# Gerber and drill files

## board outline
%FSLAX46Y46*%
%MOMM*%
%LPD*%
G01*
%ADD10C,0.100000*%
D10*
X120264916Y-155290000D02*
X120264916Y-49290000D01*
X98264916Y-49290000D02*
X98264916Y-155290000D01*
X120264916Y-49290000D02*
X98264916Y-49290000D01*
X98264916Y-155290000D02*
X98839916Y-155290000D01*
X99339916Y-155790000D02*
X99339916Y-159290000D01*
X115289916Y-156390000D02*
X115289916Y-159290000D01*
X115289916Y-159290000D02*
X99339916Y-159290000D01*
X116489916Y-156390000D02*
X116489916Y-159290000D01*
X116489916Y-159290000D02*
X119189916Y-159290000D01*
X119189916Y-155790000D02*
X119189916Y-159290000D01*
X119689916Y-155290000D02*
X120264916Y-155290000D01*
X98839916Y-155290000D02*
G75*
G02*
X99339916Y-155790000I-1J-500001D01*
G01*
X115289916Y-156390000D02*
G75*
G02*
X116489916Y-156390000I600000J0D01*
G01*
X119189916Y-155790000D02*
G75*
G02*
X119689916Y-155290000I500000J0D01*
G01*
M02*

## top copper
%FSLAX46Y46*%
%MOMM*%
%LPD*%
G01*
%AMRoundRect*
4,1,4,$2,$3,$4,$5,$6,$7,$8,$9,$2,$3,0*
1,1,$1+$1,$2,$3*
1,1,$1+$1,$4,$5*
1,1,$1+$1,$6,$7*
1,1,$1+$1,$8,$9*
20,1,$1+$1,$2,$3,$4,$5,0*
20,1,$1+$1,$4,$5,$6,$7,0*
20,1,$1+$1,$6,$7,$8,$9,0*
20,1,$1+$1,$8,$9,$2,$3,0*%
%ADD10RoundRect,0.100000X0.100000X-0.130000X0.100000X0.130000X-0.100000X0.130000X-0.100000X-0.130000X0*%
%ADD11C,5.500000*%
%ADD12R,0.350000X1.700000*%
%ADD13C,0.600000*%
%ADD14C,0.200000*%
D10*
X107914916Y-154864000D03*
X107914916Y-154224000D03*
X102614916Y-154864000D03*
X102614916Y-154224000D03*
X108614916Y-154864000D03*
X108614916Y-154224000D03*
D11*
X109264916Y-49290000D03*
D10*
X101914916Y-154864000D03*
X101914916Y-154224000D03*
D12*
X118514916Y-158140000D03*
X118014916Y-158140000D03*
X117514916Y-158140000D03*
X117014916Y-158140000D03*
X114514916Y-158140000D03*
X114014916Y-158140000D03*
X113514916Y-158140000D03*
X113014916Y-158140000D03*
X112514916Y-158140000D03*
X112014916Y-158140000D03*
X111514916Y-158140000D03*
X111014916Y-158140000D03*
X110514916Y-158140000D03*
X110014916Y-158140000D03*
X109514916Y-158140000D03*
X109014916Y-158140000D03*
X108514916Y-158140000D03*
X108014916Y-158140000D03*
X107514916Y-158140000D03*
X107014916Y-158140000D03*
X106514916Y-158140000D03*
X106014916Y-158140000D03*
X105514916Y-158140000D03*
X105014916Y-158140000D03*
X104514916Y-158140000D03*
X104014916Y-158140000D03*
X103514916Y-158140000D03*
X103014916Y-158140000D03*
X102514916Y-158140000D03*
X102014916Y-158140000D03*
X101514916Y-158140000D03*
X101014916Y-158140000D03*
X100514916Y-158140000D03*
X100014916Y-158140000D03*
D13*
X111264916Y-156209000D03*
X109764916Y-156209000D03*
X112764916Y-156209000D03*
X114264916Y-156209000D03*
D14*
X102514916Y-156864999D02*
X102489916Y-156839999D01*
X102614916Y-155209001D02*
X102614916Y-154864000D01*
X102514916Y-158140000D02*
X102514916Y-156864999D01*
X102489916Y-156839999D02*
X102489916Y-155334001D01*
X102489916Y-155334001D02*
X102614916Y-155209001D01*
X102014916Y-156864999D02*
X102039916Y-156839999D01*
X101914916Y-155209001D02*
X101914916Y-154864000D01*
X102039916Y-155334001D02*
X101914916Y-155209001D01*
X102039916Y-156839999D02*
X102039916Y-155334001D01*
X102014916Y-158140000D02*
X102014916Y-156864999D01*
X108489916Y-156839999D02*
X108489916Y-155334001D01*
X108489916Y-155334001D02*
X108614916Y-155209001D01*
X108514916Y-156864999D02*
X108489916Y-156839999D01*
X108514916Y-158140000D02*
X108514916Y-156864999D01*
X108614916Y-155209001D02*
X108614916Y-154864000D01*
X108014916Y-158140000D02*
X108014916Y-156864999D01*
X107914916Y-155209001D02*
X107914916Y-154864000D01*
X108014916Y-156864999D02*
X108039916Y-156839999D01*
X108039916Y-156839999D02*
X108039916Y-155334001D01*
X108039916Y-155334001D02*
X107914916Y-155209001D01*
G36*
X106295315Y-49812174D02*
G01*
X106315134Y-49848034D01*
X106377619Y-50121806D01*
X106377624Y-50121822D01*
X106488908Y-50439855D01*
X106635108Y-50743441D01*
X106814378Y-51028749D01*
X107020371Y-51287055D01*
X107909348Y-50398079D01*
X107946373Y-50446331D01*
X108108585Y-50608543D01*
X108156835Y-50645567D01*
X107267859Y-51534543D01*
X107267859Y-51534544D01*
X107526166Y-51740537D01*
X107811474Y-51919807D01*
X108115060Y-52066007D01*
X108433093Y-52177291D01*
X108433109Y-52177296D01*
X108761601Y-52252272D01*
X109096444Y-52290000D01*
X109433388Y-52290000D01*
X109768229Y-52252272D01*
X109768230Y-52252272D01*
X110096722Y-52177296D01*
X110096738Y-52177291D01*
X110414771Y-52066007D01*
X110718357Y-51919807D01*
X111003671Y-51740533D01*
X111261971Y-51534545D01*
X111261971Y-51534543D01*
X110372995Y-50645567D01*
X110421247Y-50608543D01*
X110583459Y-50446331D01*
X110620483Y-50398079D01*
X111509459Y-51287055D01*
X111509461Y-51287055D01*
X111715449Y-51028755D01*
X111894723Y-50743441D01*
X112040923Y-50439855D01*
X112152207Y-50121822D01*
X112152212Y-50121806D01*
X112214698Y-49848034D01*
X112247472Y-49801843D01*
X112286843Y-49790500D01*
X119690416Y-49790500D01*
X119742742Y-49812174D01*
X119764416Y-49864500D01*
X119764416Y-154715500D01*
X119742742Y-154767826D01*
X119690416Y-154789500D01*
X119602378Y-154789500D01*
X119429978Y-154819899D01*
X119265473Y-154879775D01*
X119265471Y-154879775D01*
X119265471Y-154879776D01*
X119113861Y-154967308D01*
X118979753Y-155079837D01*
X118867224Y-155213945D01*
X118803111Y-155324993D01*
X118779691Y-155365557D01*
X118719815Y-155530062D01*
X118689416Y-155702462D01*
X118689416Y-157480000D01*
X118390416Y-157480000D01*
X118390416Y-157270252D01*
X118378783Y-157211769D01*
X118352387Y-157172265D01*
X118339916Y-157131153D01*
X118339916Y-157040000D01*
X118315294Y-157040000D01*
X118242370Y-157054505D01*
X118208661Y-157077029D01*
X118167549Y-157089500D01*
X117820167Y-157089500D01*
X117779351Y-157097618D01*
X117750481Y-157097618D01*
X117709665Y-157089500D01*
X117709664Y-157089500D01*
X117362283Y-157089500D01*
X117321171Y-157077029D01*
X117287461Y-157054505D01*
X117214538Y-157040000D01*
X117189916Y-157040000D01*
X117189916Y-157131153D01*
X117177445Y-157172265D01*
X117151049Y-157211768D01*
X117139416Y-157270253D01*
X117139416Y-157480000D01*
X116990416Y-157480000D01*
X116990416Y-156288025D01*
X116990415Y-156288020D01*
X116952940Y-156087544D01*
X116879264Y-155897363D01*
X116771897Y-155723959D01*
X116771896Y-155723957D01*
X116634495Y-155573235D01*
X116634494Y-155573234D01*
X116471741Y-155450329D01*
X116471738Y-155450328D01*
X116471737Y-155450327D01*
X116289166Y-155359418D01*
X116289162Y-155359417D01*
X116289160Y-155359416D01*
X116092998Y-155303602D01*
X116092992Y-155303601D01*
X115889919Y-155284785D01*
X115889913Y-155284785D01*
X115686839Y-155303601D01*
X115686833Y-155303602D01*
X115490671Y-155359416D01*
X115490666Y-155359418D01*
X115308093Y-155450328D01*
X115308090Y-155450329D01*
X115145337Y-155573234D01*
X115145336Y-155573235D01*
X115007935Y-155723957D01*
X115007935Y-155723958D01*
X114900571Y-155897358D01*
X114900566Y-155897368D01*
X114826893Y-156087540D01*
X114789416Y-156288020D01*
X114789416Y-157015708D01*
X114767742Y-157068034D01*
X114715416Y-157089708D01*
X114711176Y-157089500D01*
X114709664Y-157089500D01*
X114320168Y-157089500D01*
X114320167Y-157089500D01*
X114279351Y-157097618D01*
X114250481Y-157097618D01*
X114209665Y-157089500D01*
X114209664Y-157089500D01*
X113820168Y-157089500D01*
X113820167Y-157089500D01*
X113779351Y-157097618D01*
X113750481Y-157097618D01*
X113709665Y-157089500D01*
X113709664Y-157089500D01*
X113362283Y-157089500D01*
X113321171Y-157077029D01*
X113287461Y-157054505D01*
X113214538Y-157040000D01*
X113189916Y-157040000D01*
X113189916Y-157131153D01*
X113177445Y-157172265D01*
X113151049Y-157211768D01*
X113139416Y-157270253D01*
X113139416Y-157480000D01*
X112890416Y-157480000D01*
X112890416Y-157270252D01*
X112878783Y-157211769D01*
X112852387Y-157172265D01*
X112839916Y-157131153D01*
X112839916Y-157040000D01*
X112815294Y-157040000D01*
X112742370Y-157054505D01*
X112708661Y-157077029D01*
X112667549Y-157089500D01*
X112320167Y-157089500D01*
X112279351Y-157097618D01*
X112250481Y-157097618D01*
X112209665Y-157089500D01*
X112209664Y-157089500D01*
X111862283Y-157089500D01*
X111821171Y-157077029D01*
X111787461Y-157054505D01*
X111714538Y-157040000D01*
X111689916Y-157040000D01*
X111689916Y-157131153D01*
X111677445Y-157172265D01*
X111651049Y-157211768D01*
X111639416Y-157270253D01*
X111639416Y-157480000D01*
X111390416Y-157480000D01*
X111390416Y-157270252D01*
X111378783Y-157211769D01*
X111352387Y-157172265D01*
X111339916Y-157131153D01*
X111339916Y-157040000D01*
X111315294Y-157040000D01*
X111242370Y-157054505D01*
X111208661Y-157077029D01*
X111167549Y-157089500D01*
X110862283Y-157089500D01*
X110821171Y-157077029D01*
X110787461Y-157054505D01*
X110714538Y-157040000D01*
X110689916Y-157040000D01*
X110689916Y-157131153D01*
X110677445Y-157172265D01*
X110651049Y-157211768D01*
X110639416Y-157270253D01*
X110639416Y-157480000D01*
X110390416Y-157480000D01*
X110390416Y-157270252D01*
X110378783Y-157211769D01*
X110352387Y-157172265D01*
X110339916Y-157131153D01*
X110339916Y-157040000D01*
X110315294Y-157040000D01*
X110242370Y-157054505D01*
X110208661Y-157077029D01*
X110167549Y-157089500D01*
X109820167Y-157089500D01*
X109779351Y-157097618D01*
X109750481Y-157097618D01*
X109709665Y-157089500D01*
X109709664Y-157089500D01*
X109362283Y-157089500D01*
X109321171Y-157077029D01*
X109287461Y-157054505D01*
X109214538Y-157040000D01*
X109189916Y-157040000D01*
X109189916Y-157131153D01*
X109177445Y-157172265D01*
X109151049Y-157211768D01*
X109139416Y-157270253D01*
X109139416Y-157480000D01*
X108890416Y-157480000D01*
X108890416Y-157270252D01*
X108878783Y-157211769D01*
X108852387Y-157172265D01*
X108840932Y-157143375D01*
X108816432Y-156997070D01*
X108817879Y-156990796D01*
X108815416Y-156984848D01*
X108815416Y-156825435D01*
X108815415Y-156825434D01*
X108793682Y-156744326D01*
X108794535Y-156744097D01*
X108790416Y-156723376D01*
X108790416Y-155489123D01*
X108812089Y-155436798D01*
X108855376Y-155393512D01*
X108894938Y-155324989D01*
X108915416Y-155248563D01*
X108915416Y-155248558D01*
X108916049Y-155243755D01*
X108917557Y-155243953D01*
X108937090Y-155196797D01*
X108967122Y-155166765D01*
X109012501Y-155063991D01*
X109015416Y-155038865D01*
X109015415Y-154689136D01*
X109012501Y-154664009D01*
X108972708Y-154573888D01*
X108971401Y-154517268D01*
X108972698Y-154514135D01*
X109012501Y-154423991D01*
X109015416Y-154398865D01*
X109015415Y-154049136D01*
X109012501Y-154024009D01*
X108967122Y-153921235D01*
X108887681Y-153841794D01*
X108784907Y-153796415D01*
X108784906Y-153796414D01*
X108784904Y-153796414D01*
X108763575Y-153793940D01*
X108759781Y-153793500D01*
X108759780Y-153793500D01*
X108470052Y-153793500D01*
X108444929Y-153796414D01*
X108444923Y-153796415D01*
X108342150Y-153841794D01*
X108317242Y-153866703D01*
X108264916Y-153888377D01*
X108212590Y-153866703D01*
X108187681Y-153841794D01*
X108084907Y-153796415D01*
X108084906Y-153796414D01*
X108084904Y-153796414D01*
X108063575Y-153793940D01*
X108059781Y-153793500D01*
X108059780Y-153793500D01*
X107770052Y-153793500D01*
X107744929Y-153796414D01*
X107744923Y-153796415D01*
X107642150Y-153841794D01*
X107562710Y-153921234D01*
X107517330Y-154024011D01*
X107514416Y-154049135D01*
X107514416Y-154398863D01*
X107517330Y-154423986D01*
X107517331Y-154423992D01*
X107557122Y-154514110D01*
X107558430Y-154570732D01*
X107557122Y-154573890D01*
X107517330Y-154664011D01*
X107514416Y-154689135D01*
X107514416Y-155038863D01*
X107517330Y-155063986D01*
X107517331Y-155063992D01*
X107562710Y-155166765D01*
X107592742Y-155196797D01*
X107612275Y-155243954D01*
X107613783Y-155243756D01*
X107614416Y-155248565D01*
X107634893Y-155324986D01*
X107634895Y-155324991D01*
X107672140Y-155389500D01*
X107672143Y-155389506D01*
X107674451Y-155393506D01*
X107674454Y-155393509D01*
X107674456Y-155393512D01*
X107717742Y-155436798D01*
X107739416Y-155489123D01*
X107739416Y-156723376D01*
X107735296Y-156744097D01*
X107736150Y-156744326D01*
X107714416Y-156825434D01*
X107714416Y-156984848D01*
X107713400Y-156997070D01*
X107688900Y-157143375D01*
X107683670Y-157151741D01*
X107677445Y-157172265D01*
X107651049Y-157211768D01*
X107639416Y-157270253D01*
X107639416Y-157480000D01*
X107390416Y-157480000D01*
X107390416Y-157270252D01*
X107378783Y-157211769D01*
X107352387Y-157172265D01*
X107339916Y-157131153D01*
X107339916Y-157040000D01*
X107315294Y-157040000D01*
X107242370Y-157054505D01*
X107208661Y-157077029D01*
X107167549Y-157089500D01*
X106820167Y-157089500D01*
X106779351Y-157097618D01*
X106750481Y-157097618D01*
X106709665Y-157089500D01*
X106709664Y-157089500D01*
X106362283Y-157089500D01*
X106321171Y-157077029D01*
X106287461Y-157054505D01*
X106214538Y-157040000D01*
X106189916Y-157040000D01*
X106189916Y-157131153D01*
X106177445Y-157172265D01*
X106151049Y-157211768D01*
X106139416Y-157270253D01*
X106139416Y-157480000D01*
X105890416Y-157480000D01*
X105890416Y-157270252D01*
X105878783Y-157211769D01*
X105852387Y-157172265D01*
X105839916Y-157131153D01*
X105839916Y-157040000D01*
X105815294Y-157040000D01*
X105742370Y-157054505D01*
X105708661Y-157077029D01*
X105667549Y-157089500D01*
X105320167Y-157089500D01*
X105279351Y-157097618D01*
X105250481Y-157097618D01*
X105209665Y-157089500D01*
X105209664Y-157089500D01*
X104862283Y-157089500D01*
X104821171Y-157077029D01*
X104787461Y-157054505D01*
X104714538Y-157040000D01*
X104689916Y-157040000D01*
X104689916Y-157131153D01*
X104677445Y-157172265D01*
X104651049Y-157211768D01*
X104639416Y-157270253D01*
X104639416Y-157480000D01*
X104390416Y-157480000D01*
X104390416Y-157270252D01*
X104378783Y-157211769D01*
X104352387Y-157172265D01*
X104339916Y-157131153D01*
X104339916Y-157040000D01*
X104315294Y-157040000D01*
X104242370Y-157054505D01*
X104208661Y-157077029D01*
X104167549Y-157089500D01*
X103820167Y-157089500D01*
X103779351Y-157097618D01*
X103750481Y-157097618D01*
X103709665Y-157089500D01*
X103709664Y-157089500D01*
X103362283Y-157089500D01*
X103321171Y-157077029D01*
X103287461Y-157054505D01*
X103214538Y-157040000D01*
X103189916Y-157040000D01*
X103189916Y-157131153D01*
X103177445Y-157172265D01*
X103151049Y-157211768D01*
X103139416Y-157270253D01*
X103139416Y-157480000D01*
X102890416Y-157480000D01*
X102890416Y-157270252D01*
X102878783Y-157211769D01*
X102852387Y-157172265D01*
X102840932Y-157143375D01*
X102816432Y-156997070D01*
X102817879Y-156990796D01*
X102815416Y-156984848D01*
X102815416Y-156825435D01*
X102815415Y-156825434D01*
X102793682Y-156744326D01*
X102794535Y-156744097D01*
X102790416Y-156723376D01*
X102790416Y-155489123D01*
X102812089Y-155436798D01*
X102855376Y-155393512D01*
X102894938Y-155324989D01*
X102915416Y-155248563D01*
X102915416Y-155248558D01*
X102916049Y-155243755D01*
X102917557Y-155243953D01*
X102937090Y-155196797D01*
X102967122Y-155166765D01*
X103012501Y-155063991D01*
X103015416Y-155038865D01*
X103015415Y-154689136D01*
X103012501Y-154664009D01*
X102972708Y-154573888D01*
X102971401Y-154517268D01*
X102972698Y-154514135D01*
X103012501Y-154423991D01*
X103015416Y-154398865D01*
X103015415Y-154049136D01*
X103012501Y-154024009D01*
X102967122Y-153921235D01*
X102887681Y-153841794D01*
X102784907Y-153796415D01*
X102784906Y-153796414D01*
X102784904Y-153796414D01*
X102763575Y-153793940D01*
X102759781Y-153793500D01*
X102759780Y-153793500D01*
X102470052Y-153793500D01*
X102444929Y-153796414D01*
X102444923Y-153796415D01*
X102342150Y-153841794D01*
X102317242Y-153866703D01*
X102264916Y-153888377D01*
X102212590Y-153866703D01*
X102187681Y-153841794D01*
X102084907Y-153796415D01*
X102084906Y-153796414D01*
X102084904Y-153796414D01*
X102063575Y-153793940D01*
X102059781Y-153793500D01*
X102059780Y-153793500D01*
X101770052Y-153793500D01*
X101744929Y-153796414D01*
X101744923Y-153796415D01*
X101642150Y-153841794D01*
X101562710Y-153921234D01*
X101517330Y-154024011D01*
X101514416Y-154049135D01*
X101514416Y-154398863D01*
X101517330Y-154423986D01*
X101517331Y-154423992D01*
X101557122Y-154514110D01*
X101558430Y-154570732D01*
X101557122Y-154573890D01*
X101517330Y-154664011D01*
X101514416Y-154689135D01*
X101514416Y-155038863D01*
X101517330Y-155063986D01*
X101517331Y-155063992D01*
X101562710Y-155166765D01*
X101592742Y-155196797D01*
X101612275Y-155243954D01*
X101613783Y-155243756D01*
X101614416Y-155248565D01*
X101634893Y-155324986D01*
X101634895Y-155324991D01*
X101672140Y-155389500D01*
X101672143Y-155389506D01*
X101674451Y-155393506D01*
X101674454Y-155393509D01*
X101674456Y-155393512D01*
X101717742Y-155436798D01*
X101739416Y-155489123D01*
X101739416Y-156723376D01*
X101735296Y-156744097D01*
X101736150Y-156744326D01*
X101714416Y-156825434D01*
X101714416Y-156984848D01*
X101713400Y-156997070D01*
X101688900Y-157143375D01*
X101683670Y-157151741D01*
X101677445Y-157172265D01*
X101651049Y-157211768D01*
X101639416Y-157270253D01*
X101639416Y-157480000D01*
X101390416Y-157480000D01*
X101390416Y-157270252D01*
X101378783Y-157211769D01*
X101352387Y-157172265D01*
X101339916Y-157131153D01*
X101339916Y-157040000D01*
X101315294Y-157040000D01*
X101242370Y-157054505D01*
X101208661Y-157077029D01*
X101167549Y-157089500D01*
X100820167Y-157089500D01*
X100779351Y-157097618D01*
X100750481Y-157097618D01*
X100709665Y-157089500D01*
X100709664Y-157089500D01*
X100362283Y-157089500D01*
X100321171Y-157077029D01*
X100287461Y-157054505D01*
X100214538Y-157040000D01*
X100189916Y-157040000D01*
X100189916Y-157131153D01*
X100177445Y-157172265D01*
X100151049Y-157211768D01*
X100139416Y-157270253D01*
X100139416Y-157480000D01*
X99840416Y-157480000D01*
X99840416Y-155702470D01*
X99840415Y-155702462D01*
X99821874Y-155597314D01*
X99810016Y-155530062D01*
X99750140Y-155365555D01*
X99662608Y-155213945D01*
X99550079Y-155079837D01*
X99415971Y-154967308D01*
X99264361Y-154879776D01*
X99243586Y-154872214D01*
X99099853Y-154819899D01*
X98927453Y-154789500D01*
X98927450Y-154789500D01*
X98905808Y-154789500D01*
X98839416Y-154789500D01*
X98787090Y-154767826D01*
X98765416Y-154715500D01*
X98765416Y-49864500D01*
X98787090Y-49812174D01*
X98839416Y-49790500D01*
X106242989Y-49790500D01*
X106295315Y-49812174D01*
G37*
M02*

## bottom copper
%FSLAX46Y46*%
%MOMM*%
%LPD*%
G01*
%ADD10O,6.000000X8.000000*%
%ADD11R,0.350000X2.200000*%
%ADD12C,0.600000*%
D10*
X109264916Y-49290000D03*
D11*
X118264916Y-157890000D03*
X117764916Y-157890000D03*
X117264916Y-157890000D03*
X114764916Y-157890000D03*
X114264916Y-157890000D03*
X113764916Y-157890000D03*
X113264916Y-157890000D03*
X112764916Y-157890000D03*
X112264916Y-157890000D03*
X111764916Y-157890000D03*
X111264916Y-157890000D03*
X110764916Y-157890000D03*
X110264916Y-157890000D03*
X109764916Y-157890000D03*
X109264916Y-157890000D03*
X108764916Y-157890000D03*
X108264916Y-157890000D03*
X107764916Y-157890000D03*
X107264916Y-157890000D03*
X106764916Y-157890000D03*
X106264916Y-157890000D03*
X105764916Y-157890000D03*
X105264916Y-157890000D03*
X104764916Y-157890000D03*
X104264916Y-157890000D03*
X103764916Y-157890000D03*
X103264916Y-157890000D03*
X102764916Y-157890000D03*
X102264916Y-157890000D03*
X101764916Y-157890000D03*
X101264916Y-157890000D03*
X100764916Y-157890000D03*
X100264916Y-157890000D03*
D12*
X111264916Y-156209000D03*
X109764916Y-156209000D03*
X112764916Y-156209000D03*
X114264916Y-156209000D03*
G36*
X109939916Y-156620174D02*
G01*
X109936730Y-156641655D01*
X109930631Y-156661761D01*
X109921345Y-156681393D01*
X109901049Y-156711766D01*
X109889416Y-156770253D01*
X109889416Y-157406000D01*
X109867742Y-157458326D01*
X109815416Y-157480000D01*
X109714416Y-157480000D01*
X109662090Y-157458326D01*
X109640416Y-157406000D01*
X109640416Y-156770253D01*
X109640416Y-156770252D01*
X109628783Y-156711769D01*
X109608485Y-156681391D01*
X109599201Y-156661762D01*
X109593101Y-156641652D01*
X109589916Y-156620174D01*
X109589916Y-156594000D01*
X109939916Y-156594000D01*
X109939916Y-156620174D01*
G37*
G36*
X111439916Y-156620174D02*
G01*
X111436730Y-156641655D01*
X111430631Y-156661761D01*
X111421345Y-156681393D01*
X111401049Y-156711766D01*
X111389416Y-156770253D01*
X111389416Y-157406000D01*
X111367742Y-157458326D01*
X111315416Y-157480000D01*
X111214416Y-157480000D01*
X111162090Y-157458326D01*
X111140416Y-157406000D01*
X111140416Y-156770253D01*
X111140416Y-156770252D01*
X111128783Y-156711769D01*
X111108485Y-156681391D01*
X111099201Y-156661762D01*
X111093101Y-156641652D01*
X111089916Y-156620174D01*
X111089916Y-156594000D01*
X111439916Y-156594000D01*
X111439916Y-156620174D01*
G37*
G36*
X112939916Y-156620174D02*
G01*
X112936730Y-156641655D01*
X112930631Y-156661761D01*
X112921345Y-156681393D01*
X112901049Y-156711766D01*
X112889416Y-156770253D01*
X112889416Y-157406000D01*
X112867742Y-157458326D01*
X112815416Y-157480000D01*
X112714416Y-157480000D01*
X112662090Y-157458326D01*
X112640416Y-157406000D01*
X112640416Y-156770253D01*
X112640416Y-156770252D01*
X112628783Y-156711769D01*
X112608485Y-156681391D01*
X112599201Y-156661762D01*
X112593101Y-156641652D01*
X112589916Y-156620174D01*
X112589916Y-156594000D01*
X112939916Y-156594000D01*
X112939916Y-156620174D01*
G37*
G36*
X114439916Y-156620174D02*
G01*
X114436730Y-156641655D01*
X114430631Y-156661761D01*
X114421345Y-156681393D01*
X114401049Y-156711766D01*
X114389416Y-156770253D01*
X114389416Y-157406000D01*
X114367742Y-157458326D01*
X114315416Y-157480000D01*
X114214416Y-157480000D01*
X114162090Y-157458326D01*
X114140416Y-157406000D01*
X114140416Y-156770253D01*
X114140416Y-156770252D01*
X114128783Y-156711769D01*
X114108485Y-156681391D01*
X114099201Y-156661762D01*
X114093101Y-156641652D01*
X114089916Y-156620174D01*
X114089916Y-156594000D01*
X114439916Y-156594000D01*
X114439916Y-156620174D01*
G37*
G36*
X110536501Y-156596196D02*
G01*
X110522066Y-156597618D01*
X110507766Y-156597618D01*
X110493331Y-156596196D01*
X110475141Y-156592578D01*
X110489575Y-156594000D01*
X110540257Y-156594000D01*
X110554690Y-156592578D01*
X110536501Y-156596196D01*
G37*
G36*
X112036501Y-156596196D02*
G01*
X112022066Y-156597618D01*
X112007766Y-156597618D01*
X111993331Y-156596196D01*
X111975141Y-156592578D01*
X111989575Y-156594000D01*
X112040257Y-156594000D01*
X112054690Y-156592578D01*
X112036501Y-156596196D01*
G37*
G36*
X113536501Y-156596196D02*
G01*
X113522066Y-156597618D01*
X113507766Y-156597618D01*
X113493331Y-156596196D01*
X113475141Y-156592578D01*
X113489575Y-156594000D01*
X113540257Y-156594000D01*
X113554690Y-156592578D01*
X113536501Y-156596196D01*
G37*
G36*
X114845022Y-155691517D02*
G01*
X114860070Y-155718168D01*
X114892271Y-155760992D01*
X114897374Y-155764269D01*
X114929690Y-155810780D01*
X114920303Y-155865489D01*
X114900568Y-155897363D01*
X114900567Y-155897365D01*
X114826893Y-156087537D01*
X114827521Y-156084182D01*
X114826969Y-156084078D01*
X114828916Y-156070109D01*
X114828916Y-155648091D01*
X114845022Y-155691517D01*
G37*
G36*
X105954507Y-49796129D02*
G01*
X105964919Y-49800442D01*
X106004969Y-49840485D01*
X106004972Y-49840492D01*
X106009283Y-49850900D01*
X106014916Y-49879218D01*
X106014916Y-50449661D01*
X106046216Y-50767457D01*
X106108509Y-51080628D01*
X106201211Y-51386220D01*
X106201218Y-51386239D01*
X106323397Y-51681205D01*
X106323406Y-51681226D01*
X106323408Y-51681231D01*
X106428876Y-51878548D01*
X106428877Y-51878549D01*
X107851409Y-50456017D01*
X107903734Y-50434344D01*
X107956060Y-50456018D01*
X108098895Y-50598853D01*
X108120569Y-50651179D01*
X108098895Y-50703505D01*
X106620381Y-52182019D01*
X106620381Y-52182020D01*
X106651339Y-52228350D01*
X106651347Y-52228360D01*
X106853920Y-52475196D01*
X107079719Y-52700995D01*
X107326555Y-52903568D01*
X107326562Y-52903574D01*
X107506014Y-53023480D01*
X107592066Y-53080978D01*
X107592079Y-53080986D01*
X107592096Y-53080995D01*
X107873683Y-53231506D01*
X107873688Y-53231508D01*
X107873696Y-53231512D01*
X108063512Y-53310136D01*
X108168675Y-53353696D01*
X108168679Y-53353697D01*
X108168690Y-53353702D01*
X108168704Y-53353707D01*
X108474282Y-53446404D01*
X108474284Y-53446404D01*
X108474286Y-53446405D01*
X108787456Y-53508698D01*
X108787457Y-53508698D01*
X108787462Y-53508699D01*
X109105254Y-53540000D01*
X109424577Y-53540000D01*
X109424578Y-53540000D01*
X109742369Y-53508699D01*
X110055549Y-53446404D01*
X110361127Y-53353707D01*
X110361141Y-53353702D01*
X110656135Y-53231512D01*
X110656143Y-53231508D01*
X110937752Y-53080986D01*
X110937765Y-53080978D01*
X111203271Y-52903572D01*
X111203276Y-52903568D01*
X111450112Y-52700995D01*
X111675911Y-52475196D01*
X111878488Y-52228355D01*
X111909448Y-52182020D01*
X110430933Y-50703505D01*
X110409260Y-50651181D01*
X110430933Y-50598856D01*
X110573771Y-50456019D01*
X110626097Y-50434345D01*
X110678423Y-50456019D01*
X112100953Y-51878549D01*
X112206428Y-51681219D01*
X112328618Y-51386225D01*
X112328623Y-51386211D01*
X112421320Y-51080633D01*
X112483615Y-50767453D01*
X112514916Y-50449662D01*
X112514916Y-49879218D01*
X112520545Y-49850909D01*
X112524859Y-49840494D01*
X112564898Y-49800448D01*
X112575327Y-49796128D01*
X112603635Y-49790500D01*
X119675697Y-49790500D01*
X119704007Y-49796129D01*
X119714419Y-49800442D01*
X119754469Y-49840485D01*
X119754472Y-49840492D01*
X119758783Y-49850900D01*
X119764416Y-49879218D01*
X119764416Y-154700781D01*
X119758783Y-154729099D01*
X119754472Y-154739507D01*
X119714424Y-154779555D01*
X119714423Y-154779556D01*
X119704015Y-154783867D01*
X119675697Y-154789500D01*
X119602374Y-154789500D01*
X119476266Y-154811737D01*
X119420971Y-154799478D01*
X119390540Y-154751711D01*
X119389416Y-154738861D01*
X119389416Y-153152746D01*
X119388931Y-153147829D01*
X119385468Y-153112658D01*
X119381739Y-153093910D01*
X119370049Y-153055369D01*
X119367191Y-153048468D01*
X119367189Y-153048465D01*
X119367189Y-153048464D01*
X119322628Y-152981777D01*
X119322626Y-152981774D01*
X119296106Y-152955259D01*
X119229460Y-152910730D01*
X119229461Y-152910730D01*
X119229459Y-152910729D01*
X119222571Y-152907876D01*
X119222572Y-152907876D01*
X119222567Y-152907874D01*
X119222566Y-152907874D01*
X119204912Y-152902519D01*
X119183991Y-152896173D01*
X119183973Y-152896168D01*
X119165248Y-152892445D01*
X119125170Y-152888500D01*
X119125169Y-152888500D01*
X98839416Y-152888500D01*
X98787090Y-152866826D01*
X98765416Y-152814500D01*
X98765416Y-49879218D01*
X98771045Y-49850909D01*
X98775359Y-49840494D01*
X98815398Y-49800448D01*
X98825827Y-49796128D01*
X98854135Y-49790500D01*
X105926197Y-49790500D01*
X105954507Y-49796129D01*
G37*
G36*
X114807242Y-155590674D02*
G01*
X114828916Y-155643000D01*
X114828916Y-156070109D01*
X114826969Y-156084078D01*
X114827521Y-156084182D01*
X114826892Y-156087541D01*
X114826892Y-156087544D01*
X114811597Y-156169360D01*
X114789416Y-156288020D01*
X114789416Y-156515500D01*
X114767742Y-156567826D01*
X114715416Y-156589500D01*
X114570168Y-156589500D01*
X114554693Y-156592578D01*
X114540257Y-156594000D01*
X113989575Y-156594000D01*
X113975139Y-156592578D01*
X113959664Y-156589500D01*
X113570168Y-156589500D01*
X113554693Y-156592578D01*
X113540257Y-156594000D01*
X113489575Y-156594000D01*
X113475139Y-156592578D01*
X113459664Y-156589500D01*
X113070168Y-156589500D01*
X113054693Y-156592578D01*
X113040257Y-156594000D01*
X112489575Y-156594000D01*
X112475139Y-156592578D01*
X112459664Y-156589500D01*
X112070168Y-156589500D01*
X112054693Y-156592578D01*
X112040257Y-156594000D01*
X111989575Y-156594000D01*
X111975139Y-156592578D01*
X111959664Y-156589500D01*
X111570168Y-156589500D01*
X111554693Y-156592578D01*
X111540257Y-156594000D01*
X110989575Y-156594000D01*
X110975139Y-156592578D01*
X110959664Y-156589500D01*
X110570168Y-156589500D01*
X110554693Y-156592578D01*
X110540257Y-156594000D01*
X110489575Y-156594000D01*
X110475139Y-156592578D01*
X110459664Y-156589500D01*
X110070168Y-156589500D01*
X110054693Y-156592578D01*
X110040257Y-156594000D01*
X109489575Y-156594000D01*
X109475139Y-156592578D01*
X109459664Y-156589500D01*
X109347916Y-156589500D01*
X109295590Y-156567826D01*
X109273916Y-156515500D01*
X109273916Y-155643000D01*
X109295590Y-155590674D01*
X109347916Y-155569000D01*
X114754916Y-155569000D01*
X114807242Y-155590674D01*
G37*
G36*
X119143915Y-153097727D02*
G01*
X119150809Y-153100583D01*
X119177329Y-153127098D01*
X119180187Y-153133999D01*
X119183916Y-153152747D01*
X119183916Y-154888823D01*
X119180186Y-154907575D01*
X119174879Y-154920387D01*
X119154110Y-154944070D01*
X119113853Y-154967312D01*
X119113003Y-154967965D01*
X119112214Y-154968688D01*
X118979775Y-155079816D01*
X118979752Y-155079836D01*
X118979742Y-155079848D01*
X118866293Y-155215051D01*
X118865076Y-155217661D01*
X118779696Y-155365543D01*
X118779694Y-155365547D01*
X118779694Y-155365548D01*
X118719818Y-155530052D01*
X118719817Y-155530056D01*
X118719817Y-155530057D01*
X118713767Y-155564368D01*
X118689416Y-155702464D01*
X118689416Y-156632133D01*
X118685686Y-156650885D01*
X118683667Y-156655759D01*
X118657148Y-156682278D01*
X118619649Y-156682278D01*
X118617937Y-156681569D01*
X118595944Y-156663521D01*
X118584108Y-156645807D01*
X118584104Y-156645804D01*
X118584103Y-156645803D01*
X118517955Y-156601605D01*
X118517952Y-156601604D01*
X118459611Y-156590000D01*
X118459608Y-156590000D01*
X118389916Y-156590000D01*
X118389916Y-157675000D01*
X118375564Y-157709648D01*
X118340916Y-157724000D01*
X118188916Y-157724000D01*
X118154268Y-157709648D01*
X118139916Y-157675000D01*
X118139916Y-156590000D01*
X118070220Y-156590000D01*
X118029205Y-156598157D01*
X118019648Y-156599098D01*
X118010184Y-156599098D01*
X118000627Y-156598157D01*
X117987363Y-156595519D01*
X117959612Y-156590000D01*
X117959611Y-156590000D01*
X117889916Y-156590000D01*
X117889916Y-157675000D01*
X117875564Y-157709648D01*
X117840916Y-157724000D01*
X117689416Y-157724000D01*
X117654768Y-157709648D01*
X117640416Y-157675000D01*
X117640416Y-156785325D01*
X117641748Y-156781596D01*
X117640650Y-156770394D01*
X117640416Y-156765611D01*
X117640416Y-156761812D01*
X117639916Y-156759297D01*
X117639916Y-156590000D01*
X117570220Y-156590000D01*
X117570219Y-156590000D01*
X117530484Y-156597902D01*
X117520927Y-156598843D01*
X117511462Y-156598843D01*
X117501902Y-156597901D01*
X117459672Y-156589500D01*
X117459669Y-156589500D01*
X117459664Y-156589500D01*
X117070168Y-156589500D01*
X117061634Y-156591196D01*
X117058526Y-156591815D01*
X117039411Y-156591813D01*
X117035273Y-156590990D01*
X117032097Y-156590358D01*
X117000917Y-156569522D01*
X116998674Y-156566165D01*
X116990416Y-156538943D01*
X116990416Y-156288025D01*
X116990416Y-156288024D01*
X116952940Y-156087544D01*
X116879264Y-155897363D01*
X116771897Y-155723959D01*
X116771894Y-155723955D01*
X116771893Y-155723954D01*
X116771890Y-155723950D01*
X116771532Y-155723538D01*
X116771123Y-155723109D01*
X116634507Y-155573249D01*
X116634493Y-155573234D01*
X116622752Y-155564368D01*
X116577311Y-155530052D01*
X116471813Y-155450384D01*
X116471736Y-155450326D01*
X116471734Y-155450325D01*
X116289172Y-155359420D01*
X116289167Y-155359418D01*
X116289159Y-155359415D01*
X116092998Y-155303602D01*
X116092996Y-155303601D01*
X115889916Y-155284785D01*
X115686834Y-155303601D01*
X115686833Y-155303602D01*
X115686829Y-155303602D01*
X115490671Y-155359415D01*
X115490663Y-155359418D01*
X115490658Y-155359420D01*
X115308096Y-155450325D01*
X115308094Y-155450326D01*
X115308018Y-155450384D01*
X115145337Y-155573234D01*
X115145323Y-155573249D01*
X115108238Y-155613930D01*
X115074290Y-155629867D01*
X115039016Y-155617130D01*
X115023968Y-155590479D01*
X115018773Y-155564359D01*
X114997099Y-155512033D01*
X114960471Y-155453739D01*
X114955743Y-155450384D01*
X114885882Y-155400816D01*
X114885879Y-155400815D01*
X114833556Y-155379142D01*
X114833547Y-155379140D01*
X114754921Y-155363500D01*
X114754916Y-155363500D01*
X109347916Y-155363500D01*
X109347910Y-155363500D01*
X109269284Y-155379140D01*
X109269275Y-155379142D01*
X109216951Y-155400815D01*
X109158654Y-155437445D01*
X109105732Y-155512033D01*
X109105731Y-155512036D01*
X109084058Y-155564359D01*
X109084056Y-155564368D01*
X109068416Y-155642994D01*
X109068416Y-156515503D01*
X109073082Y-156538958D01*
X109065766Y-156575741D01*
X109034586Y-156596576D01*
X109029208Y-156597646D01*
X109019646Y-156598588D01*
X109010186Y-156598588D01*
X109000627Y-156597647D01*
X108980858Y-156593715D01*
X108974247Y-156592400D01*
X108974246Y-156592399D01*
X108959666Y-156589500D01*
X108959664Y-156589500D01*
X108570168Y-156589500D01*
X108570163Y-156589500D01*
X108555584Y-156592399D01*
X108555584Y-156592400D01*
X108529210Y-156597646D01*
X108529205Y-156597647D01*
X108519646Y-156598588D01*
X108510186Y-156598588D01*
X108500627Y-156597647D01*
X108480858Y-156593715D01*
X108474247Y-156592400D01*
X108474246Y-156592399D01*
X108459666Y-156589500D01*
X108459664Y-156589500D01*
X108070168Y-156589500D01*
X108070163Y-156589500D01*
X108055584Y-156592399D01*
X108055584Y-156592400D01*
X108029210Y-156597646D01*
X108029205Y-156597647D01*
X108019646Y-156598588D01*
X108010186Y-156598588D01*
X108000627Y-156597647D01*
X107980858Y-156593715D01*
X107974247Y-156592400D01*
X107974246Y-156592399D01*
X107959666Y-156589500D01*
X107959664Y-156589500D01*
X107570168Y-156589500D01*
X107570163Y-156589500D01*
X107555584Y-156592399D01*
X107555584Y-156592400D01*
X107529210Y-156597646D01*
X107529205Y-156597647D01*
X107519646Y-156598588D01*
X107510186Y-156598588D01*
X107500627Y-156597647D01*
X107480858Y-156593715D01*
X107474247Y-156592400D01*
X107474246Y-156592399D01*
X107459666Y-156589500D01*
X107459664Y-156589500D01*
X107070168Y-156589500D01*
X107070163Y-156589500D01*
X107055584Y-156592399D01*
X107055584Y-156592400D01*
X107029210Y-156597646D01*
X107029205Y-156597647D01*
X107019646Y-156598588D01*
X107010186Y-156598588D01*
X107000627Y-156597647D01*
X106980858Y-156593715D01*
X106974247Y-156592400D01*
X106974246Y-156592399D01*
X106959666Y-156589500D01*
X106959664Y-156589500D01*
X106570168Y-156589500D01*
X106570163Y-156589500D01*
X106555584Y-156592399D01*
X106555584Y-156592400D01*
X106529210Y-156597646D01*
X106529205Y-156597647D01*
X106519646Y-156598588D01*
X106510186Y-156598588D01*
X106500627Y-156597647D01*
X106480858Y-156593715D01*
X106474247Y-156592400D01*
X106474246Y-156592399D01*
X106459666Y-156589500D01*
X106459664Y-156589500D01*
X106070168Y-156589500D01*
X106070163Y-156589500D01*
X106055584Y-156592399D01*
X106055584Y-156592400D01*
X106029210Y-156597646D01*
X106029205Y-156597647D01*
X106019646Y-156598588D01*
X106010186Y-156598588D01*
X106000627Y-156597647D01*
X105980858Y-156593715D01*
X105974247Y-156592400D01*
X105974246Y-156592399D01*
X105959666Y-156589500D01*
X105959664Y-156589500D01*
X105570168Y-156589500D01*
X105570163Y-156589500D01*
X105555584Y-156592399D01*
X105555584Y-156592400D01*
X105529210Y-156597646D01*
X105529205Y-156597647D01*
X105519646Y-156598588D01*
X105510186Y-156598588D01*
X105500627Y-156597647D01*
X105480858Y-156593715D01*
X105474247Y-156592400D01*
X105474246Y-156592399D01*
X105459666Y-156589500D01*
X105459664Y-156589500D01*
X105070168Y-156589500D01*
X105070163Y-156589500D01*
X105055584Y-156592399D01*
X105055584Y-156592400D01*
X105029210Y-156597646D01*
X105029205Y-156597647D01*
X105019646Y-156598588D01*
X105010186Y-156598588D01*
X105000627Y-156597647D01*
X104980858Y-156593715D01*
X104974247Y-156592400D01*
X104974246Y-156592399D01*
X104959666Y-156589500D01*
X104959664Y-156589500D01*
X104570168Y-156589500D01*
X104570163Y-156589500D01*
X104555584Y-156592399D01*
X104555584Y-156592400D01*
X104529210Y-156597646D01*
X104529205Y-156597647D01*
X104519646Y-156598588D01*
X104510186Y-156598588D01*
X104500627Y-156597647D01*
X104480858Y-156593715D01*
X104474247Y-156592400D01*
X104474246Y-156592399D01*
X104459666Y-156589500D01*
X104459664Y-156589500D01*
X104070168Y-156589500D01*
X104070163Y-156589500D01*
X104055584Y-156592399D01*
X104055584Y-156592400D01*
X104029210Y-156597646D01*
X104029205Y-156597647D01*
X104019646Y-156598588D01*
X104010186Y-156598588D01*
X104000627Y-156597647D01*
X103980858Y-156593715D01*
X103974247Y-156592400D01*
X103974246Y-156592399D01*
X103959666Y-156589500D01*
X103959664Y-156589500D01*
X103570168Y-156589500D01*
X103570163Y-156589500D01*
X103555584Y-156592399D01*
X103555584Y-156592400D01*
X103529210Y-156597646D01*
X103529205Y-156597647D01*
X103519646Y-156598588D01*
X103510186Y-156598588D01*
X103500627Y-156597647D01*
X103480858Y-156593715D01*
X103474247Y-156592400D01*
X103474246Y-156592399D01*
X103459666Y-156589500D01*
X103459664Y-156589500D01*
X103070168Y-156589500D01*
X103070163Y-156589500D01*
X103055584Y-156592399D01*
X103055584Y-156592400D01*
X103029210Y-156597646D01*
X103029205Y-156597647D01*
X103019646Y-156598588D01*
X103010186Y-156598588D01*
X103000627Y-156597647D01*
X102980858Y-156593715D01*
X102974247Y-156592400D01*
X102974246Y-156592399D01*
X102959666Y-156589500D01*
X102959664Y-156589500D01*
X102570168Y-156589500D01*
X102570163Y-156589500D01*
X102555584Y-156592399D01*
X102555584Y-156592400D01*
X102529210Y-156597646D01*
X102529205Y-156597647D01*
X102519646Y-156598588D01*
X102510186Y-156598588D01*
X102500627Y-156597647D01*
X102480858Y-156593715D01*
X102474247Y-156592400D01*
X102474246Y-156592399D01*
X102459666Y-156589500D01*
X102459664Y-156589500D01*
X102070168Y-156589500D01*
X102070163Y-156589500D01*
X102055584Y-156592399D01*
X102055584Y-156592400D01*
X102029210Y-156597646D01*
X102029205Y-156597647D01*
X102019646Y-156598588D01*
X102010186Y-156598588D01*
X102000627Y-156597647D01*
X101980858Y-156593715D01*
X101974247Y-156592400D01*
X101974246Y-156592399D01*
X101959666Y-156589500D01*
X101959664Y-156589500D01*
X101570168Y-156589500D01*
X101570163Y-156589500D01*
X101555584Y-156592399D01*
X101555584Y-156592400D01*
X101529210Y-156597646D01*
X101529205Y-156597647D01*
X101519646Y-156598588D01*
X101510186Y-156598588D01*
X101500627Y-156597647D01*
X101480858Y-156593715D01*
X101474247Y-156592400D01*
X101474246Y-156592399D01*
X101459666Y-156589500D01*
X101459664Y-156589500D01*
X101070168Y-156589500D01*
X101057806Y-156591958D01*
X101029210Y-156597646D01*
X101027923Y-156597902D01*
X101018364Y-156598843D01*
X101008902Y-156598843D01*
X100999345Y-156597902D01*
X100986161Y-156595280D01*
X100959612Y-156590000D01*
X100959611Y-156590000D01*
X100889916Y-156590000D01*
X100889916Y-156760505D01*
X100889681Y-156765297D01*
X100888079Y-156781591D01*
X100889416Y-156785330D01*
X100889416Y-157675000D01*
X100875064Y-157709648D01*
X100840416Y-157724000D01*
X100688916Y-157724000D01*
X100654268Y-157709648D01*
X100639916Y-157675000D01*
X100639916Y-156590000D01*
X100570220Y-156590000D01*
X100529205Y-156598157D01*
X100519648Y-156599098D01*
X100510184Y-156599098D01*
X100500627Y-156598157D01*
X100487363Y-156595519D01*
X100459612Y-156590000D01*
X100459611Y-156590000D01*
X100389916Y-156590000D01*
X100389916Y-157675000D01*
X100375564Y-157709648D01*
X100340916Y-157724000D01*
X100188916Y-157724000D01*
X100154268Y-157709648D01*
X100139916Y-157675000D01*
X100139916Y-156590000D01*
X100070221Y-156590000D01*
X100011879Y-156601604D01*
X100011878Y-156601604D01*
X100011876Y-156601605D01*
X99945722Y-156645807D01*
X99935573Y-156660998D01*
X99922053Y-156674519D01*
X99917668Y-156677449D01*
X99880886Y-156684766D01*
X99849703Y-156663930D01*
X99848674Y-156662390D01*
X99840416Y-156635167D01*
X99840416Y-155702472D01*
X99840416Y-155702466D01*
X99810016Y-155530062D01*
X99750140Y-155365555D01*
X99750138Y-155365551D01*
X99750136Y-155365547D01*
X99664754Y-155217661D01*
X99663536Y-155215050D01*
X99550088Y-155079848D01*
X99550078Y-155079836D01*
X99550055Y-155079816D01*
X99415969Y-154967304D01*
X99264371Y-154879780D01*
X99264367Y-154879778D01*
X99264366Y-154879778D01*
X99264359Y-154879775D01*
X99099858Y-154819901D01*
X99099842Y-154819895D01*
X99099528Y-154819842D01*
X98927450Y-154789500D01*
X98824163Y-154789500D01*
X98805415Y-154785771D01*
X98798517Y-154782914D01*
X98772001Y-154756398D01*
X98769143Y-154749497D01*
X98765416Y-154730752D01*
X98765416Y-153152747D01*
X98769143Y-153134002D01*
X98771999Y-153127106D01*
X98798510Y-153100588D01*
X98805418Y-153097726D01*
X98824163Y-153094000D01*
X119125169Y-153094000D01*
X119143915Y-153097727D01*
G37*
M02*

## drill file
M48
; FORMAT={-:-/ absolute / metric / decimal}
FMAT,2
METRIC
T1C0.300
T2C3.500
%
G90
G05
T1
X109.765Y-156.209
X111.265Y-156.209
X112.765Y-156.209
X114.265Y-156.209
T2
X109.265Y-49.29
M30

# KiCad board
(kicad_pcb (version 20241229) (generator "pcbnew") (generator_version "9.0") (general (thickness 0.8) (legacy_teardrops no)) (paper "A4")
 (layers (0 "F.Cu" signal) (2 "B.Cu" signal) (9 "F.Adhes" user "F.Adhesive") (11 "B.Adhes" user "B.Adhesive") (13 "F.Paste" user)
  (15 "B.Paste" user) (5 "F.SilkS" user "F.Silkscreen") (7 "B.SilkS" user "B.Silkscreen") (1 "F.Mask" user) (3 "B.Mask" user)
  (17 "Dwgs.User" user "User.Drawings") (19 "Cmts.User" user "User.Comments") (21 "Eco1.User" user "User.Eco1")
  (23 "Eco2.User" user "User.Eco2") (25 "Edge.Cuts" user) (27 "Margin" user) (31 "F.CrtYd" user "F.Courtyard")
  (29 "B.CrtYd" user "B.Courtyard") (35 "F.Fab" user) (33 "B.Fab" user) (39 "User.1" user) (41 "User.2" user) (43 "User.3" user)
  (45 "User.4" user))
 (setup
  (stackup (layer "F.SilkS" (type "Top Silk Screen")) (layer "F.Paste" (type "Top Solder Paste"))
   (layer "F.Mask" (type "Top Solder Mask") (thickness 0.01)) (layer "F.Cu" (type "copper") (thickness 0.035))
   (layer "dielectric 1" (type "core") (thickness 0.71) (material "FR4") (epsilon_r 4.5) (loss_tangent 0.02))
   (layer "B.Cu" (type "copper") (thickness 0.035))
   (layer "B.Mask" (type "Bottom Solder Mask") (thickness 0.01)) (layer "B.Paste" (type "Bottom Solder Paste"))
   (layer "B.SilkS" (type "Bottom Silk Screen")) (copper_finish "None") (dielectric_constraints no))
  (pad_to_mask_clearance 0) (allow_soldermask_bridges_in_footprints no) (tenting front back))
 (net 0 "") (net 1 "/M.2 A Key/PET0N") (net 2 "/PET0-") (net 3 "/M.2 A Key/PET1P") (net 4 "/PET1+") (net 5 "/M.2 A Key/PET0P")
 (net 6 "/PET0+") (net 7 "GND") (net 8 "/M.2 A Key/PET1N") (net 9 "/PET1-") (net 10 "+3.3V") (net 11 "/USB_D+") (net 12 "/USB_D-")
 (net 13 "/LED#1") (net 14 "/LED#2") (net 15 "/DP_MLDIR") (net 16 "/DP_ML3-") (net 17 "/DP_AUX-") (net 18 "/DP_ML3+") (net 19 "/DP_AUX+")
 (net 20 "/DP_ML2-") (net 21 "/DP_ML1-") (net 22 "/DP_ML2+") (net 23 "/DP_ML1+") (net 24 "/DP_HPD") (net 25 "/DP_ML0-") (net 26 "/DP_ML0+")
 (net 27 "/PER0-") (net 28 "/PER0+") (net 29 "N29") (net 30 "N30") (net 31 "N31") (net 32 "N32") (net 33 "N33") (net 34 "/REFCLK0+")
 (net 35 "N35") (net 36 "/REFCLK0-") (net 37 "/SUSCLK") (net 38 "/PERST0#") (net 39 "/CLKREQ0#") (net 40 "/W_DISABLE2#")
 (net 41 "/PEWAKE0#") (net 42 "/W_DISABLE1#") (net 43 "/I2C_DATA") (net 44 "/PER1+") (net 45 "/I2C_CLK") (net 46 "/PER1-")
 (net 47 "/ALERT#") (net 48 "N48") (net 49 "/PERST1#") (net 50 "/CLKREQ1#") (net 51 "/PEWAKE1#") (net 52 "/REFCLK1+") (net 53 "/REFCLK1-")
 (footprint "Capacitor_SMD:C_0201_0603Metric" (layer "F.Cu") (at 107.914916 154.544 90)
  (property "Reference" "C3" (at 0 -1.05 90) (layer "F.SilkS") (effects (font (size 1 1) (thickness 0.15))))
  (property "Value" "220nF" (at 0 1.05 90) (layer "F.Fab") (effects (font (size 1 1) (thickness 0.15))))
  (pad "" smd roundrect (at -0.345 0 90) (size 0.318 0.36) (layers "F.Paste") (roundrect_rratio 0.25))
  (pad "" smd roundrect (at 0.345 0 90) (size 0.318 0.36) (layers "F.Paste") (roundrect_rratio 0.25))
  (pad "1" smd roundrect (at -0.32 0 90) (size 0.46 0.4) (layers "F.Cu" "F.Mask") (roundrect_rratio 0.25) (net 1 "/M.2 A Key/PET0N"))
  (pad "2" smd roundrect (at 0.32 0 90) (size 0.46 0.4) (layers "F.Cu" "F.Mask") (roundrect_rratio 0.25) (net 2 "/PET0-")))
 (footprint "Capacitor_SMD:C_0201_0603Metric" (layer "F.Cu") (at 102.614916 154.544 90)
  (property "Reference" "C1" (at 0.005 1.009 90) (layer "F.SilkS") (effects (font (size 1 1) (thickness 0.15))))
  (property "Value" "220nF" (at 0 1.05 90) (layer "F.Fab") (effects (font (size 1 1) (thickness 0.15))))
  (pad "" smd roundrect (at -0.345 0 90) (size 0.318 0.36) (layers "F.Paste") (roundrect_rratio 0.25))
  (pad "" smd roundrect (at 0.345 0 90) (size 0.318 0.36) (layers "F.Paste") (roundrect_rratio 0.25))
  (pad "1" smd roundrect (at -0.32 0 90) (size 0.46 0.4) (layers "F.Cu" "F.Mask") (roundrect_rratio 0.25) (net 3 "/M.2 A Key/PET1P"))
  (pad "2" smd roundrect (at 0.32 0 90) (size 0.46 0.4) (layers "F.Cu" "F.Mask") (roundrect_rratio 0.25) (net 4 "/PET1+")))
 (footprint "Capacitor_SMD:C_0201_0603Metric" (layer "F.Cu") (at 108.614916 154.544 90)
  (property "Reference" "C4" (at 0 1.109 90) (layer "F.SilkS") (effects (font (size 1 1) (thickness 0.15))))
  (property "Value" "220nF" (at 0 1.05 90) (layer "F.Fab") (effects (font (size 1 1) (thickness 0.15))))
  (pad "" smd roundrect (at -0.345 0 90) (size 0.318 0.36) (layers "F.Paste") (roundrect_rratio 0.25))
  (pad "" smd roundrect (at 0.345 0 90) (size 0.318 0.36) (layers "F.Paste") (roundrect_rratio 0.25))
  (pad "1" smd roundrect (at -0.32 0 90) (size 0.46 0.4) (layers "F.Cu" "F.Mask") (roundrect_rratio 0.25) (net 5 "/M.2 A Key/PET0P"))
  (pad "2" smd roundrect (at 0.32 0 90) (size 0.46 0.4) (layers "F.Cu" "F.Mask") (roundrect_rratio 0.25) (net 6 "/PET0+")))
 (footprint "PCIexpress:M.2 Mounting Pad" (layer "F.Cu") (at 109.264916 129.29)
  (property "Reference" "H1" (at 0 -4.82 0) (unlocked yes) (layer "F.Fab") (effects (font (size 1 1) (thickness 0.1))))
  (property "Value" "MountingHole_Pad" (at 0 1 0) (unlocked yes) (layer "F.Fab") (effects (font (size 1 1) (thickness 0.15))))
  (pad "1" thru_hole circle (at 0 -80) (size 5.5 5.5) (drill 3.5) (layers "*.Cu" "*.Mask") (remove_unused_layers no) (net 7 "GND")
   (padstack (mode front_inner_back)
    (layer "Inner" (shape circle) (size 5.5 5.5) (zone_connect -1))
    (layer "B.Cu" (shape oval) (size 6 8) (thermal_bridge_angle 45) (zone_connect -1)))))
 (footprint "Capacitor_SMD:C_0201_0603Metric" (layer "F.Cu") (at 101.914916 154.544 90)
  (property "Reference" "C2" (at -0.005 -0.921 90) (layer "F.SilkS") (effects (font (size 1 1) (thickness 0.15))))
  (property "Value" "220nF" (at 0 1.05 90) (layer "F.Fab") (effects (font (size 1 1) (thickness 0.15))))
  (pad "" smd roundrect (at -0.345 0 90) (size 0.318 0.36) (layers "F.Paste") (roundrect_rratio 0.25))
  (pad "" smd roundrect (at 0.345 0 90) (size 0.318 0.36) (layers "F.Paste") (roundrect_rratio 0.25))
  (pad "1" smd roundrect (at -0.32 0 90) (size 0.46 0.4) (layers "F.Cu" "F.Mask") (roundrect_rratio 0.25) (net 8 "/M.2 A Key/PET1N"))
  (pad "2" smd roundrect (at 0.32 0 90) (size 0.46 0.4) (layers "F.Cu" "F.Mask") (roundrect_rratio 0.25) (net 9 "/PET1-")))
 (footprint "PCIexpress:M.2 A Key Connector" (layer "F.Cu") (at 109.264916 158.18)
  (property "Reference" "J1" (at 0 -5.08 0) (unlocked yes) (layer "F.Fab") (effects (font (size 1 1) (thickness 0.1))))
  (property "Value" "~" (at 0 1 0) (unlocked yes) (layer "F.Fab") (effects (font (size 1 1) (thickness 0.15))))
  (fp_line (start -11 -2.89) (end -10.425 -2.89) (stroke (width 0.1) (type default)) (layer "Edge.Cuts"))
  (fp_line (start -9.925 -2.39) (end -9.925 1.11) (stroke (width 0.1) (type default)) (layer "Edge.Cuts"))
  (fp_line (start 6.025 -1.79) (end 6.025 1.11) (stroke (width 0.1) (type default)) (layer "Edge.Cuts"))
  (fp_line (start 6.025 1.11) (end -9.925 1.11) (stroke (width 0.1) (type default)) (layer "Edge.Cuts"))
  (fp_line (start 7.225 -1.79) (end 7.225 1.11) (stroke (width 0.1) (type default)) (layer "Edge.Cuts"))
  (fp_line (start 7.225 1.11) (end 9.925 1.11) (stroke (width 0.1) (type default)) (layer "Edge.Cuts"))
  (fp_line (start 9.925 -2.39) (end 9.925 1.11) (stroke (width 0.1) (type default)) (layer "Edge.Cuts"))
  (fp_line (start 10.425 -2.89) (end 11 -2.89) (stroke (width 0.1) (type default)) (layer "Edge.Cuts"))
  (fp_arc (start -10.425 -2.89) (mid -10.071447 -2.743553) (end -9.925 -2.39) (stroke (width 0.1) (type default)) (layer "Edge.Cuts"))
  (fp_arc (start 6.025 -1.79) (mid 6.625 -2.39) (end 7.225 -1.79) (stroke (width 0.1) (type default)) (layer "Edge.Cuts"))
  (fp_arc (start 9.925 -2.39) (mid 10.071447 -2.743553) (end 10.425 -2.89) (stroke (width 0.1) (type default)) (layer "Edge.Cuts"))
  (pad "1" smd rect (at 9.25 -0.04 180) (size 0.35 1.7) (layers "F.Cu") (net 7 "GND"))
  (pad "2" smd rect (at 9 -0.29 180) (size 0.35 2.2) (layers "B.Cu") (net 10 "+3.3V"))
  (pad "3" smd rect (at 8.75 -0.04 180) (size 0.35 1.7) (layers "F.Cu") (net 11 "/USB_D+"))
  (pad "4" smd rect (at 8.5 -0.29 180) (size 0.35 2.2) (layers "B.Cu") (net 10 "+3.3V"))
  (pad "5" smd rect (at 8.25 -0.04 180) (size 0.35 1.7) (layers "F.Cu") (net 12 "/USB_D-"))
  (pad "6" smd rect (at 8 -0.29 180) (size 0.35 2.2) (layers "B.Cu") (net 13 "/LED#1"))
  (pad "7" smd rect (at 7.75 -0.04 180) (size 0.35 1.7) (layers "F.Cu") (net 7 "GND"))
  (pad "16" smd rect (at 5.5 -0.29 180) (size 0.35 2.2) (layers "B.Cu") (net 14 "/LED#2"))
  (pad "17" smd rect (at 5.25 -0.04 180) (size 0.35 1.7) (layers "F.Cu") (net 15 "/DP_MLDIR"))
  (pad "18" smd rect (at 5 -0.29 180) (size 0.35 2.2) (layers "B.Cu") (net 7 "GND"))
  (pad "19" smd rect (at 4.75 -0.04 180) (size 0.35 1.7) (layers "F.Cu") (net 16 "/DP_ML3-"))
  (pad "20" smd rect (at 4.5 -0.29 180) (size 0.35 2.2) (layers "B.Cu") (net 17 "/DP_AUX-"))
  (pad "21" smd rect (at 4.25 -0.04 180) (size 0.35 1.7) (layers "F.Cu") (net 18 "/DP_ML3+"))
  (pad "22" smd rect (at 4 -0.29 180) (size 0.35 2.2) (layers "B.Cu") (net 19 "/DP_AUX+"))
  (pad "23" smd rect (at 3.75 -0.04 180) (size 0.35 1.7) (layers "F.Cu") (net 7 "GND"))
  (pad "24" smd rect (at 3.5 -0.29 180) (size 0.35 2.2) (layers "B.Cu") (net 7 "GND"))
  (pad "25" smd rect (at 3.25 -0.04 180) (size 0.35 1.7) (layers "F.Cu") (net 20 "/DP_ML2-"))
  (pad "26" smd rect (at 3 -0.29 180) (size 0.35 2.2) (layers "B.Cu") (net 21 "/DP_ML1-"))
  (pad "27" smd rect (at 2.75 -0.04 180) (size 0.35 1.7) (layers "F.Cu") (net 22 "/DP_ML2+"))
  (pad "28" smd rect (at 2.5 -0.29 180) (size 0.35 2.2) (layers "B.Cu") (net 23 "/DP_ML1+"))
  (pad "29" smd rect (at 2.25 -0.04 180) (size 0.35 1.7) (layers "F.Cu") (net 7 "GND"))
  (pad "30" smd rect (at 2 -0.29 180) (size 0.35 2.2) (layers "B.Cu") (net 7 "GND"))
  (pad "31" smd rect (at 1.75 -0.04 180) (size 0.35 1.7) (layers "F.Cu") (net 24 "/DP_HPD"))
  (pad "32" smd rect (at 1.5 -0.29 180) (size 0.35 2.2) (layers "B.Cu") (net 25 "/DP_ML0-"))
  (pad "33" smd rect (at 1.25 -0.04 180) (size 0.35 1.7) (layers "F.Cu") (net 7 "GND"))
  (pad "34" smd rect (at 1 -0.29 180) (size 0.35 2.2) (layers "B.Cu") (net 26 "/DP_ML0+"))
  (pad "35" smd rect (at 0.75 -0.04 180) (size 0.35 1.7) (layers "F.Cu") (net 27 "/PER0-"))
  (pad "36" smd rect (at 0.5 -0.29 180) (size 0.35 2.2) (layers "B.Cu") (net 7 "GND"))
  (pad "37" smd rect (at 0.25 -0.04 180) (size 0.35 1.7) (layers "F.Cu") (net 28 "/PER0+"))
  (pad "38" smd rect (at 0 -0.29 180) (size 0.35 2.2) (layers "B.Cu") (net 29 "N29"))
  (pad "39" smd rect (at -0.25 -0.04 180) (size 0.35 1.7) (layers "F.Cu") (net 7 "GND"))
  (pad "40" smd rect (at -0.5 -0.29 180) (size 0.35 2.2) (layers "B.Cu") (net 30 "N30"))
  (pad "41" smd rect (at -0.75 -0.04 180) (size 0.35 1.7) (layers "F.Cu") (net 5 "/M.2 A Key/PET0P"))
  (pad "42" smd rect (at -1 -0.29 180) (size 0.35 2.2) (layers "B.Cu") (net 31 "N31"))
  (pad "43" smd rect (at -1.25 -0.04 180) (size 0.35 1.7) (layers "F.Cu") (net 1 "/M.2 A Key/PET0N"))
  (pad "44" smd rect (at -1.5 -0.29 180) (size 0.35 2.2) (layers "B.Cu") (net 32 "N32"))
  (pad "45" smd rect (at -1.75 -0.04 180) (size 0.35 1.7) (layers "F.Cu") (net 7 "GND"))
  (pad "46" smd rect (at -2 -0.29 180) (size 0.35 2.2) (layers "B.Cu") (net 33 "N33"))
  (pad "47" smd rect (at -2.25 -0.04 180) (size 0.35 1.7) (layers "F.Cu") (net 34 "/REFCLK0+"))
  (pad "48" smd rect (at -2.5 -0.29 180) (size 0.35 2.2) (layers "B.Cu") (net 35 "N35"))
  (pad "49" smd rect (at -2.75 -0.04 180) (size 0.35 1.7) (layers "F.Cu") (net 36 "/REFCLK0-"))
  (pad "50" smd rect (at -3 -0.29 180) (size 0.35 2.2) (layers "B.Cu") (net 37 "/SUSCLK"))
  (pad "51" smd rect (at -3.25 -0.04 180) (size 0.35 1.7) (layers "F.Cu") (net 7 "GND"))
  (pad "52" smd rect (at -3.5 -0.29 180) (size 0.35 2.2) (layers "B.Cu") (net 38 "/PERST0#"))
  (pad "53" smd rect (at -3.75 -0.04 180) (size 0.35 1.7) (layers "F.Cu") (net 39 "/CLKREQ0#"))
  (pad "54" smd rect (at -4 -0.29 180) (size 0.35 2.2) (layers "B.Cu") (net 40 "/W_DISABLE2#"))
  (pad "55" smd rect (at -4.25 -0.04 180) (size 0.35 1.7) (layers "F.Cu") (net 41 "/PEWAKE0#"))
  (pad "56" smd rect (at -4.5 -0.29 180) (size 0.35 2.2) (layers "B.Cu") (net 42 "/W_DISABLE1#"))
  (pad "57" smd rect (at -4.75 -0.04 180) (size 0.35 1.7) (layers "F.Cu") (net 7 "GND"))
  (pad "58" smd rect (at -5 -0.29 180) (size 0.35 2.2) (layers "B.Cu") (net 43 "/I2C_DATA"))
  (pad "59" smd rect (at -5.25 -0.04 180) (size 0.35 1.7) (layers "F.Cu") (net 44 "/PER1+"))
  (pad "60" smd rect (at -5.5 -0.29 180) (size 0.35 2.2) (layers "B.Cu") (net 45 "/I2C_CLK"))
  (pad "61" smd rect (at -5.75 -0.04 180) (size 0.35 1.7) (layers "F.Cu") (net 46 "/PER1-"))
  (pad "62" smd rect (at -6 -0.29 180) (size 0.35 2.2) (layers "B.Cu") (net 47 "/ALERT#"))
  (pad "63" smd rect (at -6.25 -0.04 180) (size 0.35 1.7) (layers "F.Cu") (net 7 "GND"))
  (pad "64" smd rect (at -6.5 -0.29 180) (size 0.35 2.2) (layers "B.Cu") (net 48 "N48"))
  (pad "65" smd rect (at -6.75 -0.04 180) (size 0.35 1.7) (layers "F.Cu") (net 3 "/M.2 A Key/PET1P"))
  (pad "66" smd rect (at -7 -0.29 180) (size 0.35 2.2) (layers "B.Cu") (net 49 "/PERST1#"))
  (pad "67" smd rect (at -7.25 -0.04 180) (size 0.35 1.7) (layers "F.Cu") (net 8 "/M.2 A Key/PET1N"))
  (pad "68" smd rect (at -7.5 -0.29 180) (size 0.35 2.2) (layers "B.Cu") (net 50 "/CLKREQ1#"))
  (pad "69" smd rect (at -7.75 -0.04 180) (size 0.35 1.7) (layers "F.Cu") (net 7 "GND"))
  (pad "70" smd rect (at -8 -0.29 180) (size 0.35 2.2) (layers "B.Cu") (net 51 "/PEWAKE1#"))
  (pad "71" smd rect (at -8.25 -0.04 180) (size 0.35 1.7) (layers "F.Cu") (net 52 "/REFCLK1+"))
  (pad "72" smd rect (at -8.5 -0.29 180) (size 0.35 2.2) (layers "B.Cu") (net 10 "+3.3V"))
  (pad "73" smd rect (at -8.75 -0.04 180) (size 0.35 1.7) (layers "F.Cu") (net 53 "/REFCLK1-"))
  (pad "74" smd rect (at -9 -0.29 180) (size 0.35 2.2) (layers "B.Cu") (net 10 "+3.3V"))
  (pad "75" smd rect (at -9.25 -0.04 180) (size 0.35 1.7) (layers "F.Cu") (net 7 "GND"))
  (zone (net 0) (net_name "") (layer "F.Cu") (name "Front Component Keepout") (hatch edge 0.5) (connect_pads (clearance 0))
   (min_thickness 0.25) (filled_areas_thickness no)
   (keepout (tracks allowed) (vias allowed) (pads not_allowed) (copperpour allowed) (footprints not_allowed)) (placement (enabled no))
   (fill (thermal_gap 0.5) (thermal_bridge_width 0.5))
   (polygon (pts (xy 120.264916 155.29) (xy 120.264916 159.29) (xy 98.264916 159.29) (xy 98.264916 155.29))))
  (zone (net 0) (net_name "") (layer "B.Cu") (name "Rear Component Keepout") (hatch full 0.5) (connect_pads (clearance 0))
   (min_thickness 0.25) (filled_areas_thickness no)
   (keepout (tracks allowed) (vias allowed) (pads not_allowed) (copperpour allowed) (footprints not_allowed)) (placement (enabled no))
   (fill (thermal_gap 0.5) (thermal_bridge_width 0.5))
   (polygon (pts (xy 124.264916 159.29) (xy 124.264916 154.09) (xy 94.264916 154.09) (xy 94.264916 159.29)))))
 (gr_line (start 120.264916 155.29) (end 120.264916 49.29) (stroke (width 0.1) (type default)) (layer "Edge.Cuts"))
 (gr_line (start 98.264916 49.29) (end 98.264916 155.29) (stroke (width 0.1) (type default)) (layer "Edge.Cuts"))
 (gr_line (start 120.264916 49.29) (end 98.264916 49.29) (stroke (width 0.1) (type solid)) (layer "Edge.Cuts"))
 (via (at 111.264916 156.209) (size 0.6) (drill 0.3) (layers "F.Cu" "B.Cu") (free yes) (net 7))
 (via (at 109.764916 156.209) (size 0.6) (drill 0.3) (layers "F.Cu" "B.Cu") (free yes) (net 7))
 (via (at 112.764916 156.209) (size 0.6) (drill 0.3) (layers "F.Cu" "B.Cu") (free yes) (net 7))
 (via (at 114.264916 156.209) (size 0.6) (drill 0.3) (layers "F.Cu" "B.Cu") (free yes) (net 7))
 (segment (start 102.514916 156.864999) (end 102.489916 156.839999) (width 0.2) (layer "F.Cu") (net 3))
 (segment (start 102.614916 155.209001) (end 102.614916 154.864) (width 0.2) (layer "F.Cu") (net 3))
 (segment (start 102.514916 158.14) (end 102.514916 156.864999) (width 0.2) (layer "F.Cu") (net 3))
 (segment (start 102.489916 156.839999) (end 102.489916 155.334001) (width 0.2) (layer "F.Cu") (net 3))
 (segment (start 102.489916 155.334001) (end 102.614916 155.209001) (width 0.2) (layer "F.Cu") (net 3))
 (segment (start 102.014916 156.864999) (end 102.039916 156.839999) (width 0.2) (layer "F.Cu") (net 8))
 (segment (start 101.914916 155.209001) (end 101.914916 154.864) (width 0.2) (layer "F.Cu") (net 8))
 (segment (start 102.039916 155.334001) (end 101.914916 155.209001) (width 0.2) (layer "F.Cu") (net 8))
 (segment (start 102.039916 156.839999) (end 102.039916 155.334001) (width 0.2) (layer "F.Cu") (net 8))
 (segment (start 102.014916 158.14) (end 102.014916 156.864999) (width 0.2) (layer "F.Cu") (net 8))
 (segment (start 108.489916 156.839999) (end 108.489916 155.334001) (width 0.2) (layer "F.Cu") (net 5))
 (segment (start 108.489916 155.334001) (end 108.614916 155.209001) (width 0.2) (layer "F.Cu") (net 5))
 (segment (start 108.514916 156.864999) (end 108.489916 156.839999) (width 0.2) (layer "F.Cu") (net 5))
 (segment (start 108.514916 158.14) (end 108.514916 156.864999) (width 0.2) (layer "F.Cu") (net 5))
 (segment (start 108.614916 155.209001) (end 108.614916 154.864) (width 0.2) (layer "F.Cu") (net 5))
 (segment (start 108.014916 158.14) (end 108.014916 156.864999) (width 0.2) (layer "F.Cu") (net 1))
 (segment (start 107.914916 155.209001) (end 107.914916 154.864) (width 0.2) (layer "F.Cu") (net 1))
 (segment (start 108.014916 156.864999) (end 108.039916 156.839999) (width 0.2) (layer "F.Cu") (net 1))
 (segment (start 108.039916 156.839999) (end 108.039916 155.334001) (width 0.2) (layer "F.Cu") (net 1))
 (segment (start 108.039916 155.334001) (end 107.914916 155.209001) (width 0.2) (layer "F.Cu") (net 1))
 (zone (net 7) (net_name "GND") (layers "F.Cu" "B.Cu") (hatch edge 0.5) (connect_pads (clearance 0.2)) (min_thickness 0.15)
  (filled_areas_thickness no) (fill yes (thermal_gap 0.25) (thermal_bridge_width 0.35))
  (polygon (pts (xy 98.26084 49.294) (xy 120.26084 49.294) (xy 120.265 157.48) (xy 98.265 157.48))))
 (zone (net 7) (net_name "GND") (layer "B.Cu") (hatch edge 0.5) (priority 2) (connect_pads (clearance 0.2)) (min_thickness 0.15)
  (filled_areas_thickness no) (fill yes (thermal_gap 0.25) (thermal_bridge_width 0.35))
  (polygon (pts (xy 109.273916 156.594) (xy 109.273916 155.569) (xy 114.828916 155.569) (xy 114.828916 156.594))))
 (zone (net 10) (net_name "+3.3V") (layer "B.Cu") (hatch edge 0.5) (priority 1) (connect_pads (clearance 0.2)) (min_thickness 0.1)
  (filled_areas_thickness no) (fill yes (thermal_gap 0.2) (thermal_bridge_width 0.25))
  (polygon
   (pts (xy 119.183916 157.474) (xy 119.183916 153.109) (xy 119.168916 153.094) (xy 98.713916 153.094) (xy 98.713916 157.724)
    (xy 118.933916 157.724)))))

